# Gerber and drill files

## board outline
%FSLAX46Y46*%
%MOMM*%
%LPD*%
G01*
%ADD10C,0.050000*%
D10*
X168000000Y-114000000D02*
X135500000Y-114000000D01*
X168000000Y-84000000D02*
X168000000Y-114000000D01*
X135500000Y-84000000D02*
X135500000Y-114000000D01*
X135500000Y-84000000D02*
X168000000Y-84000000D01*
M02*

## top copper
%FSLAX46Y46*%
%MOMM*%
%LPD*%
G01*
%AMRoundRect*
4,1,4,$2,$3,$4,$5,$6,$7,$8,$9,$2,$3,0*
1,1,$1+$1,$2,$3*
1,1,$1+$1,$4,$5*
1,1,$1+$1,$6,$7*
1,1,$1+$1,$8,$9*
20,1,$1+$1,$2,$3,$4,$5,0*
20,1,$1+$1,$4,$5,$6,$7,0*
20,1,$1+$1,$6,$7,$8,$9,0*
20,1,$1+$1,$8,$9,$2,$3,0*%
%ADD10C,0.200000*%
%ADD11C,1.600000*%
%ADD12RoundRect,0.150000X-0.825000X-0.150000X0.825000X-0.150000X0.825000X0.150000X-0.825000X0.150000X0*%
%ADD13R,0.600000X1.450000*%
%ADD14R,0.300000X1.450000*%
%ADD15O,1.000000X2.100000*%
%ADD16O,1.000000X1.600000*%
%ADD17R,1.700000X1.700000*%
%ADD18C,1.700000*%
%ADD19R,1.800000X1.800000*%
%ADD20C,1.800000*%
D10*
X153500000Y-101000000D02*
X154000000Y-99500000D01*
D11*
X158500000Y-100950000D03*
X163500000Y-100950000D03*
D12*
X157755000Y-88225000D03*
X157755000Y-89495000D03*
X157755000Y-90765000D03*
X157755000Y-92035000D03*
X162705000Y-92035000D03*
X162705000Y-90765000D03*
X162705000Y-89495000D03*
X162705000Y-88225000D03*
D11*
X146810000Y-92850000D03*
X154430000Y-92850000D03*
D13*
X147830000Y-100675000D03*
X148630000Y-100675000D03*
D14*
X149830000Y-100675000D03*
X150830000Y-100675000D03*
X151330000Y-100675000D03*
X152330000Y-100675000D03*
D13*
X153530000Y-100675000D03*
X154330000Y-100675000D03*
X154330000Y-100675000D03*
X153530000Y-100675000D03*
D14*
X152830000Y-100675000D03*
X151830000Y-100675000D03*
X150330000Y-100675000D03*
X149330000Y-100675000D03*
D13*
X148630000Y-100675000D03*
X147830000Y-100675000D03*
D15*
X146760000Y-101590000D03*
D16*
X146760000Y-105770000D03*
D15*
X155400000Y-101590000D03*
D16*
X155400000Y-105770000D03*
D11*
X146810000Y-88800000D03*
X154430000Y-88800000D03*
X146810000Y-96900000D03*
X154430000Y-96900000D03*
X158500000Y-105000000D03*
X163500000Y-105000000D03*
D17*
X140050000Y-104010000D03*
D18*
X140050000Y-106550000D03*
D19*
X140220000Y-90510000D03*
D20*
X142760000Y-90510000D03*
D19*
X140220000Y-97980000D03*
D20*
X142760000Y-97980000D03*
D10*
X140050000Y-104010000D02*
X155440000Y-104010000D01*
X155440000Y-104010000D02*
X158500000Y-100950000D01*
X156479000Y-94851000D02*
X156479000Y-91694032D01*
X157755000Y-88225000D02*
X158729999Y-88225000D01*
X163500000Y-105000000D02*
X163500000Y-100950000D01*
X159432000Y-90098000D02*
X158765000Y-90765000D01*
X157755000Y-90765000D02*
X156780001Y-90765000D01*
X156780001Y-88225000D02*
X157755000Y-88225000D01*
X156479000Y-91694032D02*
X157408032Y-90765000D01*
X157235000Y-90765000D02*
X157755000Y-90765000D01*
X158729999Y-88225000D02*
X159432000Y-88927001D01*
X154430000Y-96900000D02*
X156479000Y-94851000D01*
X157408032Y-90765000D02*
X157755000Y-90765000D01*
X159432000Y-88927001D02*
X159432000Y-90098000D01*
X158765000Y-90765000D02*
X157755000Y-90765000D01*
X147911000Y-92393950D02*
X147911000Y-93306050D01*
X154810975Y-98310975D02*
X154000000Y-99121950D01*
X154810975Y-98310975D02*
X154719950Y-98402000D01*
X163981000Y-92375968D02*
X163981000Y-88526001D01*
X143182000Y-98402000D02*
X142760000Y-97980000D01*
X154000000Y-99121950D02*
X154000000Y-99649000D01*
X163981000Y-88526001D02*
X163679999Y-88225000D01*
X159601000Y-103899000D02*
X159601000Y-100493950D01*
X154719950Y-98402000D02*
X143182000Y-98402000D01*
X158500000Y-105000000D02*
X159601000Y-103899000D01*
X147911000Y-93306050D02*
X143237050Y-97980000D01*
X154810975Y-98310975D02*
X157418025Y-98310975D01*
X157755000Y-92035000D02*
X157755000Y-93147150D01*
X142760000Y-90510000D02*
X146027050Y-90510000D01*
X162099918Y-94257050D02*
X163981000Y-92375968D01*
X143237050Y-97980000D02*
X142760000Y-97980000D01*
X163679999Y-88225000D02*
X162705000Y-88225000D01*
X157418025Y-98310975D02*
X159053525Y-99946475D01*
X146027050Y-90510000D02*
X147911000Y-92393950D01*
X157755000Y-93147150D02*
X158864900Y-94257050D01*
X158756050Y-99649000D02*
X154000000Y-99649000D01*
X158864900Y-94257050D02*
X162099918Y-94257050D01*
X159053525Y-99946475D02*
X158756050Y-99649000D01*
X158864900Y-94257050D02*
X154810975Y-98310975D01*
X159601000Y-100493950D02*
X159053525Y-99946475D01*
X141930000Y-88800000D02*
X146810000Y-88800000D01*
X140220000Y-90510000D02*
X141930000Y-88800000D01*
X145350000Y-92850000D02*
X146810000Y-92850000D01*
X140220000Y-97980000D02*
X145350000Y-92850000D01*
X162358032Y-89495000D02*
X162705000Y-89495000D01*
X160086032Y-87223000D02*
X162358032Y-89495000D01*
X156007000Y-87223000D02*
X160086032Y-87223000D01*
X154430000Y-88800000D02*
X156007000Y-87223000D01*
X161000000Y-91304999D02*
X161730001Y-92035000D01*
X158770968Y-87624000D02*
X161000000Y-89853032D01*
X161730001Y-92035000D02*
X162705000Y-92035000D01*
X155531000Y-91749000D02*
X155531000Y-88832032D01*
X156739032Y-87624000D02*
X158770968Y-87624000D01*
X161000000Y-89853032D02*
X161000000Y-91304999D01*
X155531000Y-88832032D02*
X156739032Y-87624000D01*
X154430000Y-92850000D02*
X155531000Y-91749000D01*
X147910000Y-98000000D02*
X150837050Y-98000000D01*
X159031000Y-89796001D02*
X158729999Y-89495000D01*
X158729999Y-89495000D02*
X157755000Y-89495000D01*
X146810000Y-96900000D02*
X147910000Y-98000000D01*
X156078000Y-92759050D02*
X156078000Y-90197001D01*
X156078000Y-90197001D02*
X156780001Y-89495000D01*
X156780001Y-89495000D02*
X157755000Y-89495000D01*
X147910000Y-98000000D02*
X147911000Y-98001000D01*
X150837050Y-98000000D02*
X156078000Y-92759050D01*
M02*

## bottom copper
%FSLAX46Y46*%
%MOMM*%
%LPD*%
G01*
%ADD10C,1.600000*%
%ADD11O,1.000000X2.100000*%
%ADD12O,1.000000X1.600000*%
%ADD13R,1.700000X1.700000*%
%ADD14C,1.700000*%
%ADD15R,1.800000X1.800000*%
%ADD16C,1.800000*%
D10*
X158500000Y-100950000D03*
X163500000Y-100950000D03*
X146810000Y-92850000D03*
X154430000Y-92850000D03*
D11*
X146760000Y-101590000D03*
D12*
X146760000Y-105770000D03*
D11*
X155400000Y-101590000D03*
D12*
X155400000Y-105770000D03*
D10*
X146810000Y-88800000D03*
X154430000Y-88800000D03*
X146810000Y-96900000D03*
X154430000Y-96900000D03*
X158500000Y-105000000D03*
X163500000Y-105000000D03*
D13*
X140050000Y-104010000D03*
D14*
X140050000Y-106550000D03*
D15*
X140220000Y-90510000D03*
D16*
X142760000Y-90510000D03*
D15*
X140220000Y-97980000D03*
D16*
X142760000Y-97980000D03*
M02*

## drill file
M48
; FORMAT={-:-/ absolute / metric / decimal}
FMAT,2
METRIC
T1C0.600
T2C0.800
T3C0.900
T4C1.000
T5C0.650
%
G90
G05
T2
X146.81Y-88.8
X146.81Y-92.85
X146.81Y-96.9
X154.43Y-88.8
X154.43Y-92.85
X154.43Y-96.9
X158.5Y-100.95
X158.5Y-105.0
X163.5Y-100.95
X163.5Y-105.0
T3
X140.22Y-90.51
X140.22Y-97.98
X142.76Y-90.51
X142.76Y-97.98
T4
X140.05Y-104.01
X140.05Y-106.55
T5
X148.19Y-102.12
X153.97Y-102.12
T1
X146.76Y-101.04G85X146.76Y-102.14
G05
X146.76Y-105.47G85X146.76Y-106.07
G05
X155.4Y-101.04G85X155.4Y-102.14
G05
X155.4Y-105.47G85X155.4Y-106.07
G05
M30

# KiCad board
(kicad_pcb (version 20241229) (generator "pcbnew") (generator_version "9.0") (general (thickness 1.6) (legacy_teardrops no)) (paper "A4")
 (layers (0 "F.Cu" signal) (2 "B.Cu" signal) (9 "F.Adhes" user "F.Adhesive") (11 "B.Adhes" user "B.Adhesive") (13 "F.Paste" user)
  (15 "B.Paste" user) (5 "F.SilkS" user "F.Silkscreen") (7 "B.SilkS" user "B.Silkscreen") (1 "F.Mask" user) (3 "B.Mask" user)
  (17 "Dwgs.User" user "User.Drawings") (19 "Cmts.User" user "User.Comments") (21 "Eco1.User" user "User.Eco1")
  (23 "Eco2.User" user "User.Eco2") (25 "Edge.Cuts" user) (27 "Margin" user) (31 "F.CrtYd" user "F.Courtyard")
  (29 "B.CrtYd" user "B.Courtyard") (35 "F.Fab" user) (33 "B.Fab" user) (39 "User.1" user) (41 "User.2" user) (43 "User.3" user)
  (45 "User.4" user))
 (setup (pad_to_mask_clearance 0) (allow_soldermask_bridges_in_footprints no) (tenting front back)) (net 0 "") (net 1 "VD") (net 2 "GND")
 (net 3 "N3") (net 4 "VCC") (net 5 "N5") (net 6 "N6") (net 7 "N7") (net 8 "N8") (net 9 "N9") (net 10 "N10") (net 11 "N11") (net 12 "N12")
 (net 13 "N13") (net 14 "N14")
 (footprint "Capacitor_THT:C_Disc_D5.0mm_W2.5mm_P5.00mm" (layer "F.Cu") (at 158.5 100.95)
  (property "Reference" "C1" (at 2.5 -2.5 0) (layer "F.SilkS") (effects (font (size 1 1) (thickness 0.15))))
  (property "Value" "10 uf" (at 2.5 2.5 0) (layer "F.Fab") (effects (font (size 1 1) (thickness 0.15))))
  (pad "1" thru_hole circle (at 0 0) (size 1.6 1.6) (drill 0.8) (layers "*.Cu" "*.Mask") (remove_unused_layers no) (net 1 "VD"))
  (pad "2" thru_hole circle (at 5 0) (size 1.6 1.6) (drill 0.8) (layers "*.Cu" "*.Mask") (remove_unused_layers no) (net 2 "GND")))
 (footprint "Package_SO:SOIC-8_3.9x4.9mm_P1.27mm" (layer "F.Cu") (at 160.23 90.13)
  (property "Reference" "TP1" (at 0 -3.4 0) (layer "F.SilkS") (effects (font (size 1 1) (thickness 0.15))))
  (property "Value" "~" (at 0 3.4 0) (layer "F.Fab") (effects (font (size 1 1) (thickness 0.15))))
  (pad "1" smd roundrect (at -2.475 -1.905) (size 1.95 0.6) (layers "F.Cu" "F.Mask" "F.Paste") (roundrect_rratio 0.25) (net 2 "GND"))
  (pad "2" smd roundrect (at -2.475 -0.635) (size 1.95 0.6) (layers "F.Cu" "F.Mask" "F.Paste") (roundrect_rratio 0.25) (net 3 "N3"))
  (pad "3" smd roundrect (at -2.475 0.635) (size 1.95 0.6) (layers "F.Cu" "F.Mask" "F.Paste") (roundrect_rratio 0.25) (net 2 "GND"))
  (pad "4" smd roundrect (at -2.475 1.905) (size 1.95 0.6) (layers "F.Cu" "F.Mask" "F.Paste") (roundrect_rratio 0.25) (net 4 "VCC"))
  (pad "5" smd roundrect (at 2.475 1.905) (size 1.95 0.6) (layers "F.Cu" "F.Mask" "F.Paste") (roundrect_rratio 0.25) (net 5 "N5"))
  (pad "6" smd roundrect (at 2.475 0.635) (size 1.95 0.6) (layers "F.Cu" "F.Mask" "F.Paste") (roundrect_rratio 0.25))
  (pad "7" smd roundrect (at 2.475 -0.635) (size 1.95 0.6) (layers "F.Cu" "F.Mask" "F.Paste") (roundrect_rratio 0.25) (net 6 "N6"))
  (pad "8" smd roundrect (at 2.475 -1.905) (size 1.95 0.6) (layers "F.Cu" "F.Mask" "F.Paste") (roundrect_rratio 0.25) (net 4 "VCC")))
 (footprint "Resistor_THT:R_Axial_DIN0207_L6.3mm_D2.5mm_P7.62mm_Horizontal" (layer "F.Cu") (at 146.81 92.85)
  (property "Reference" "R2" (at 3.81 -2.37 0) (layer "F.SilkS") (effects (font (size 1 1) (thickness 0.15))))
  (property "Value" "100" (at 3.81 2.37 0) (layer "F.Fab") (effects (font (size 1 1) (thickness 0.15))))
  (pad "1" thru_hole circle (at 0 0) (size 1.6 1.6) (drill 0.8) (layers "*.Cu" "*.Mask") (remove_unused_layers no) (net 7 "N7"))
  (pad "2" thru_hole circle (at 7.62 0) (size 1.6 1.6) (drill 0.8) (layers "*.Cu" "*.Mask") (remove_unused_layers no) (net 5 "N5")))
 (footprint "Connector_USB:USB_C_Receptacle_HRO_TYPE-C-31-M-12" (layer "F.Cu") (at 151.08 104.72)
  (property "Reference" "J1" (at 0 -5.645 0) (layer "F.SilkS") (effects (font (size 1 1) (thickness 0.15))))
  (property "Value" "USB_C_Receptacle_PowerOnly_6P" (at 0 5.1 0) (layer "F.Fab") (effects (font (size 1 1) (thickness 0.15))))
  (pad "" np_thru_hole circle (at -2.89 -2.6) (size 0.65 0.65) (drill 0.65) (layers "*.Cu" "*.Mask"))
  (pad "" np_thru_hole circle (at 2.89 -2.6) (size 0.65 0.65) (drill 0.65) (layers "*.Cu" "*.Mask"))
  (pad "A1" smd rect (at -3.25 -4.045) (size 0.6 1.45) (layers "F.Cu" "F.Mask" "F.Paste"))
  (pad "A4" smd rect (at -2.45 -4.045) (size 0.6 1.45) (layers "F.Cu" "F.Mask" "F.Paste"))
  (pad "A5" smd rect (at -1.25 -4.045) (size 0.3 1.45) (layers "F.Cu" "F.Mask" "F.Paste") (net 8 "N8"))
  (pad "A6" smd rect (at -0.25 -4.045) (size 0.3 1.45) (layers "F.Cu" "F.Mask" "F.Paste"))
  (pad "A7" smd rect (at 0.25 -4.045) (size 0.3 1.45) (layers "F.Cu" "F.Mask" "F.Paste"))
  (pad "A8" smd rect (at 1.25 -4.045) (size 0.3 1.45) (layers "F.Cu" "F.Mask" "F.Paste"))
  (pad "A9" smd rect (at 2.45 -4.045) (size 0.6 1.45) (layers "F.Cu" "F.Mask" "F.Paste") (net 4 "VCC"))
  (pad "A12" smd rect (at 3.25 -4.045) (size 0.6 1.45) (layers "F.Cu" "F.Mask" "F.Paste") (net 2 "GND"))
  (pad "B1" smd rect (at 3.25 -4.045) (size 0.6 1.45) (layers "F.Cu" "F.Mask" "F.Paste"))
  (pad "B4" smd rect (at 2.45 -4.045) (size 0.6 1.45) (layers "F.Cu" "F.Mask" "F.Paste"))
  (pad "B5" smd rect (at 1.75 -4.045) (size 0.3 1.45) (layers "F.Cu" "F.Mask" "F.Paste") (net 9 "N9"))
  (pad "B6" smd rect (at 0.75 -4.045) (size 0.3 1.45) (layers "F.Cu" "F.Mask" "F.Paste"))
  (pad "B7" smd rect (at -0.75 -4.045) (size 0.3 1.45) (layers "F.Cu" "F.Mask" "F.Paste"))
  (pad "B8" smd rect (at -1.75 -4.045) (size 0.3 1.45) (layers "F.Cu" "F.Mask" "F.Paste"))
  (pad "B9" smd rect (at -2.45 -4.045) (size 0.6 1.45) (layers "F.Cu" "F.Mask" "F.Paste") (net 4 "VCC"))
  (pad "B12" smd rect (at -3.25 -4.045) (size 0.6 1.45) (layers "F.Cu" "F.Mask" "F.Paste") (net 2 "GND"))
  (pad "S1" thru_hole oval (at -4.32 -3.13) (size 1 2.1) (drill oval 0.6 1.7) (layers "*.Cu" "*.Mask") (remove_unused_layers no)
   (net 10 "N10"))
  (pad "S1" thru_hole oval (at -4.32 1.05) (size 1 1.6) (drill oval 0.6 1.2) (layers "*.Cu" "*.Mask") (remove_unused_layers no)
   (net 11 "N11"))
  (pad "S1" thru_hole oval (at 4.32 -3.13) (size 1 2.1) (drill oval 0.6 1.7) (layers "*.Cu" "*.Mask") (remove_unused_layers no)
   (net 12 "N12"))
  (pad "S1" thru_hole oval (at 4.32 1.05) (size 1 1.6) (drill oval 0.6 1.2) (layers "*.Cu" "*.Mask") (remove_unused_layers no)
   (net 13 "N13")))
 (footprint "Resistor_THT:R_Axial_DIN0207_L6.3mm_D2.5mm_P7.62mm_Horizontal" (layer "F.Cu") (at 146.81 88.8)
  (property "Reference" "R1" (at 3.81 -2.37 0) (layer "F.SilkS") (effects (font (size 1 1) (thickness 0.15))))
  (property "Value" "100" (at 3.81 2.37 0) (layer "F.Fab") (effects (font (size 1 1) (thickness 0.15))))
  (pad "1" thru_hole circle (at 0 0) (size 1.6 1.6) (drill 0.8) (layers "*.Cu" "*.Mask") (remove_unused_layers no) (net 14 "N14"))
  (pad "2" thru_hole circle (at 7.62 0) (size 1.6 1.6) (drill 0.8) (layers "*.Cu" "*.Mask") (remove_unused_layers no) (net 6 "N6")))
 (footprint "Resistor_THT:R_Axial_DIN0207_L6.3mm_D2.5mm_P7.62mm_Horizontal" (layer "F.Cu") (at 146.81 96.9)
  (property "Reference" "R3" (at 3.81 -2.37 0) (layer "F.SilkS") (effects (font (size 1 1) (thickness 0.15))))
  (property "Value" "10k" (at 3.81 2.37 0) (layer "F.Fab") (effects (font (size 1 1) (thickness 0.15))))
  (pad "1" thru_hole circle (at 0 0) (size 1.6 1.6) (drill 0.8) (layers "*.Cu" "*.Mask") (remove_unused_layers no) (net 3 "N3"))
  (pad "2" thru_hole circle (at 7.62 0) (size 1.6 1.6) (drill 0.8) (layers "*.Cu" "*.Mask") (remove_unused_layers no) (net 2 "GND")))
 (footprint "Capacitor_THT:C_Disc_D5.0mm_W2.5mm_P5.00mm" (layer "F.Cu") (at 158.5 105)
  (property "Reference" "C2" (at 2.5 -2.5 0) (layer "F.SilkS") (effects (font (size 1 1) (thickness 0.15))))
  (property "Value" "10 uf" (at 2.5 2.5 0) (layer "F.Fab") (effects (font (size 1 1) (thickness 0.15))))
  (pad "1" thru_hole circle (at 0 0) (size 1.6 1.6) (drill 0.8) (layers "*.Cu" "*.Mask") (remove_unused_layers no) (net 4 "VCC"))
  (pad "2" thru_hole circle (at 5 0) (size 1.6 1.6) (drill 0.8) (layers "*.Cu" "*.Mask") (remove_unused_layers no) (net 2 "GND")))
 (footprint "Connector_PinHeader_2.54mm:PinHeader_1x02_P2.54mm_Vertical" (layer "F.Cu") (at 140.05 104.01)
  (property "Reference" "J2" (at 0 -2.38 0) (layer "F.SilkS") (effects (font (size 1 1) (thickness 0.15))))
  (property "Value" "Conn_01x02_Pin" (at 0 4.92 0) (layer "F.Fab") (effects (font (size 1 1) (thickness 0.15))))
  (pad "1" thru_hole rect (at 0 0) (size 1.7 1.7) (drill 1) (layers "*.Cu" "*.Mask") (remove_unused_layers no) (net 1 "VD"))
  (pad "2" thru_hole circle (at 0 2.54) (size 1.7 1.7) (drill 1) (layers "*.Cu" "*.Mask") (remove_unused_layers no) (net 2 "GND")))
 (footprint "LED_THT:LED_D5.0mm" (layer "F.Cu") (at 140.22 90.51)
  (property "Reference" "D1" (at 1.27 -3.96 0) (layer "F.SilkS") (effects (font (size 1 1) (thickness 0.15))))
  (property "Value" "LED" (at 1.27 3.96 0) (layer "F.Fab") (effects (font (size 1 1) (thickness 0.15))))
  (pad "1" thru_hole rect (at 0 0) (size 1.8 1.8) (drill 0.9) (layers "*.Cu" "*.Mask") (remove_unused_layers no) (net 14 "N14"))
  (pad "2" thru_hole circle (at 2.54 0) (size 1.8 1.8) (drill 0.9) (layers "*.Cu" "*.Mask") (remove_unused_layers no) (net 4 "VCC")))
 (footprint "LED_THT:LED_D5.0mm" (layer "F.Cu") (at 140.22 97.98)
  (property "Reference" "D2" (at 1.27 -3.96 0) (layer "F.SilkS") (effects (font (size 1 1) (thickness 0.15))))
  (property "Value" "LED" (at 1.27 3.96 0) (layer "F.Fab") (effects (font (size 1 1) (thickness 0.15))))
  (pad "1" thru_hole rect (at 0 0) (size 1.8 1.8) (drill 0.9) (layers "*.Cu" "*.Mask") (remove_unused_layers no) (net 7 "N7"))
  (pad "2" thru_hole circle (at 2.54 0) (size 1.8 1.8) (drill 0.9) (layers "*.Cu" "*.Mask") (remove_unused_layers no) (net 4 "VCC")))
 (gr_line (start 153.5 101) (end 154 99.5) (stroke (width 0.2) (type default)) (layer "F.Cu") (net 4))
 (gr_line (start 168 114) (end 135.5 114) (stroke (width 0.05) (type default)) (layer "Edge.Cuts"))
 (gr_line (start 168 84) (end 168 114) (stroke (width 0.05) (type default)) (layer "Edge.Cuts"))
 (gr_line (start 135.5 84) (end 135.5 114) (stroke (width 0.05) (type default)) (layer "Edge.Cuts"))
 (gr_line (start 135.5 84) (end 168 84) (stroke (width 0.05) (type default)) (layer "Edge.Cuts"))
 (segment (start 140.05 104.01) (end 155.44 104.01) (width 0.2) (layer "F.Cu") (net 1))
 (segment (start 155.44 104.01) (end 158.5 100.95) (width 0.2) (layer "F.Cu") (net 1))
 (segment (start 156.479 94.851) (end 156.479 91.694032) (width 0.2) (layer "F.Cu") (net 2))
 (segment (start 157.755 88.225) (end 158.729999 88.225) (width 0.2) (layer "F.Cu") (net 2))
 (segment (start 163.5 105) (end 163.5 100.95) (width 0.2) (layer "F.Cu") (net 2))
 (segment (start 159.432 90.098) (end 158.765 90.765) (width 0.2) (layer "F.Cu") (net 2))
 (segment (start 157.755 90.765) (end 156.780001 90.765) (width 0.2) (layer "F.Cu") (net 2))
 (segment (start 156.780001 88.225) (end 157.755 88.225) (width 0.2) (layer "F.Cu") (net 2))
 (segment (start 156.479 91.694032) (end 157.408032 90.765) (width 0.2) (layer "F.Cu") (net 2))
 (segment (start 157.235 90.765) (end 157.755 90.765) (width 0.2) (layer "F.Cu") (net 2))
 (segment (start 158.729999 88.225) (end 159.432 88.927001) (width 0.2) (layer "F.Cu") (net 2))
 (segment (start 154.43 96.9) (end 156.479 94.851) (width 0.2) (layer "F.Cu") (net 2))
 (segment (start 157.408032 90.765) (end 157.755 90.765) (width 0.2) (layer "F.Cu") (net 2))
 (segment (start 159.432 88.927001) (end 159.432 90.098) (width 0.2) (layer "F.Cu") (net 2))
 (segment (start 158.765 90.765) (end 157.755 90.765) (width 0.2) (layer "F.Cu") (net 2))
 (segment (start 147.911 92.39395) (end 147.911 93.30605) (width 0.2) (layer "F.Cu") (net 4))
 (segment (start 154.810975 98.310975) (end 154 99.12195) (width 0.2) (layer "F.Cu") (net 4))
 (segment (start 154.810975 98.310975) (end 154.71995 98.402) (width 0.2) (layer "F.Cu") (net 4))
 (segment (start 163.981 92.375968) (end 163.981 88.526001) (width 0.2) (layer "F.Cu") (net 4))
 (segment (start 143.182 98.402) (end 142.76 97.98) (width 0.2) (layer "F.Cu") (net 4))
 (segment (start 154 99.12195) (end 154 99.649) (width 0.2) (layer "F.Cu") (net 4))
 (segment (start 163.981 88.526001) (end 163.679999 88.225) (width 0.2) (layer "F.Cu") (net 4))
 (segment (start 159.601 103.899) (end 159.601 100.49395) (width 0.2) (layer "F.Cu") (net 4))
 (segment (start 154.71995 98.402) (end 143.182 98.402) (width 0.2) (layer "F.Cu") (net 4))
 (segment (start 158.5 105) (end 159.601 103.899) (width 0.2) (layer "F.Cu") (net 4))
 (segment (start 147.911 93.30605) (end 143.23705 97.98) (width 0.2) (layer "F.Cu") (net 4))
 (segment (start 154.810975 98.310975) (end 157.418025 98.310975) (width 0.2) (layer "F.Cu") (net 4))
 (segment (start 157.755 92.035) (end 157.755 93.14715) (width 0.2) (layer "F.Cu") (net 4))
 (segment (start 142.76 90.51) (end 146.02705 90.51) (width 0.2) (layer "F.Cu") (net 4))
 (segment (start 162.099918 94.25705) (end 163.981 92.375968) (width 0.2) (layer "F.Cu") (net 4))
 (segment (start 143.23705 97.98) (end 142.76 97.98) (width 0.2) (layer "F.Cu") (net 4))
 (segment (start 163.679999 88.225) (end 162.705 88.225) (width 0.2) (layer "F.Cu") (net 4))
 (segment (start 157.418025 98.310975) (end 159.053525 99.946475) (width 0.2) (layer "F.Cu") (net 4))
 (segment (start 146.02705 90.51) (end 147.911 92.39395) (width 0.2) (layer "F.Cu") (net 4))
 (segment (start 157.755 93.14715) (end 158.8649 94.25705) (width 0.2) (layer "F.Cu") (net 4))
 (segment (start 158.75605 99.649) (end 154 99.649) (width 0.2) (layer "F.Cu") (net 4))
 (segment (start 158.8649 94.25705) (end 162.099918 94.25705) (width 0.2) (layer "F.Cu") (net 4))
 (segment (start 159.053525 99.946475) (end 158.75605 99.649) (width 0.2) (layer "F.Cu") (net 4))
 (segment (start 158.8649 94.25705) (end 154.810975 98.310975) (width 0.2) (layer "F.Cu") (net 4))
 (segment (start 159.601 100.49395) (end 159.053525 99.946475) (width 0.2) (layer "F.Cu") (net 4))
 (segment (start 141.93 88.8) (end 146.81 88.8) (width 0.2) (layer "F.Cu") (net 14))
 (segment (start 140.22 90.51) (end 141.93 88.8) (width 0.2) (layer "F.Cu") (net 14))
 (segment (start 145.35 92.85) (end 146.81 92.85) (width 0.2) (layer "F.Cu") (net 7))
 (segment (start 140.22 97.98) (end 145.35 92.85) (width 0.2) (layer "F.Cu") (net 7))
 (segment (start 162.358032 89.495) (end 162.705 89.495) (width 0.2) (layer "F.Cu") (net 6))
 (segment (start 160.086032 87.223) (end 162.358032 89.495) (width 0.2) (layer "F.Cu") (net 6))
 (segment (start 156.007 87.223) (end 160.086032 87.223) (width 0.2) (layer "F.Cu") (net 6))
 (segment (start 154.43 88.8) (end 156.007 87.223) (width 0.2) (layer "F.Cu") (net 6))
 (segment (start 161 91.304999) (end 161.730001 92.035) (width 0.2) (layer "F.Cu") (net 5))
 (segment (start 158.770968 87.624) (end 161 89.853032) (width 0.2) (layer "F.Cu") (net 5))
 (segment (start 161.730001 92.035) (end 162.705 92.035) (width 0.2) (layer "F.Cu") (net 5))
 (segment (start 155.531 91.749) (end 155.531 88.832032) (width 0.2) (layer "F.Cu") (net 5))
 (segment (start 156.739032 87.624) (end 158.770968 87.624) (width 0.2) (layer "F.Cu") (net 5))
 (segment (start 161 89.853032) (end 161 91.304999) (width 0.2) (layer "F.Cu") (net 5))
 (segment (start 155.531 88.832032) (end 156.739032 87.624) (width 0.2) (layer "F.Cu") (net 5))
 (segment (start 154.43 92.85) (end 155.531 91.749) (width 0.2) (layer "F.Cu") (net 5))
 (segment (start 147.91 98) (end 150.83705 98) (width 0.2) (layer "F.Cu") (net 3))
 (segment (start 159.031 89.796001) (end 158.729999 89.495) (width 0.2) (layer "F.Cu") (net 3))
 (segment (start 158.729999 89.495) (end 157.755 89.495) (width 0.2) (layer "F.Cu") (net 3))
 (segment (start 146.81 96.9) (end 147.91 98) (width 0.2) (layer "F.Cu") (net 3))
 (segment (start 156.078 92.75905) (end 156.078 90.197001) (width 0.2) (layer "F.Cu") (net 3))
 (segment (start 156.078 90.197001) (end 156.780001 89.495) (width 0.2) (layer "F.Cu") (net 3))
 (segment (start 156.780001 89.495) (end 157.755 89.495) (width 0.2) (layer "F.Cu") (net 3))
 (segment (start 147.91 98) (end 147.911 98.001) (width 0.2) (layer "F.Cu") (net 3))
 (segment (start 150.83705 98) (end 156.078 92.75905) (width 0.2) (layer "F.Cu") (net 3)))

